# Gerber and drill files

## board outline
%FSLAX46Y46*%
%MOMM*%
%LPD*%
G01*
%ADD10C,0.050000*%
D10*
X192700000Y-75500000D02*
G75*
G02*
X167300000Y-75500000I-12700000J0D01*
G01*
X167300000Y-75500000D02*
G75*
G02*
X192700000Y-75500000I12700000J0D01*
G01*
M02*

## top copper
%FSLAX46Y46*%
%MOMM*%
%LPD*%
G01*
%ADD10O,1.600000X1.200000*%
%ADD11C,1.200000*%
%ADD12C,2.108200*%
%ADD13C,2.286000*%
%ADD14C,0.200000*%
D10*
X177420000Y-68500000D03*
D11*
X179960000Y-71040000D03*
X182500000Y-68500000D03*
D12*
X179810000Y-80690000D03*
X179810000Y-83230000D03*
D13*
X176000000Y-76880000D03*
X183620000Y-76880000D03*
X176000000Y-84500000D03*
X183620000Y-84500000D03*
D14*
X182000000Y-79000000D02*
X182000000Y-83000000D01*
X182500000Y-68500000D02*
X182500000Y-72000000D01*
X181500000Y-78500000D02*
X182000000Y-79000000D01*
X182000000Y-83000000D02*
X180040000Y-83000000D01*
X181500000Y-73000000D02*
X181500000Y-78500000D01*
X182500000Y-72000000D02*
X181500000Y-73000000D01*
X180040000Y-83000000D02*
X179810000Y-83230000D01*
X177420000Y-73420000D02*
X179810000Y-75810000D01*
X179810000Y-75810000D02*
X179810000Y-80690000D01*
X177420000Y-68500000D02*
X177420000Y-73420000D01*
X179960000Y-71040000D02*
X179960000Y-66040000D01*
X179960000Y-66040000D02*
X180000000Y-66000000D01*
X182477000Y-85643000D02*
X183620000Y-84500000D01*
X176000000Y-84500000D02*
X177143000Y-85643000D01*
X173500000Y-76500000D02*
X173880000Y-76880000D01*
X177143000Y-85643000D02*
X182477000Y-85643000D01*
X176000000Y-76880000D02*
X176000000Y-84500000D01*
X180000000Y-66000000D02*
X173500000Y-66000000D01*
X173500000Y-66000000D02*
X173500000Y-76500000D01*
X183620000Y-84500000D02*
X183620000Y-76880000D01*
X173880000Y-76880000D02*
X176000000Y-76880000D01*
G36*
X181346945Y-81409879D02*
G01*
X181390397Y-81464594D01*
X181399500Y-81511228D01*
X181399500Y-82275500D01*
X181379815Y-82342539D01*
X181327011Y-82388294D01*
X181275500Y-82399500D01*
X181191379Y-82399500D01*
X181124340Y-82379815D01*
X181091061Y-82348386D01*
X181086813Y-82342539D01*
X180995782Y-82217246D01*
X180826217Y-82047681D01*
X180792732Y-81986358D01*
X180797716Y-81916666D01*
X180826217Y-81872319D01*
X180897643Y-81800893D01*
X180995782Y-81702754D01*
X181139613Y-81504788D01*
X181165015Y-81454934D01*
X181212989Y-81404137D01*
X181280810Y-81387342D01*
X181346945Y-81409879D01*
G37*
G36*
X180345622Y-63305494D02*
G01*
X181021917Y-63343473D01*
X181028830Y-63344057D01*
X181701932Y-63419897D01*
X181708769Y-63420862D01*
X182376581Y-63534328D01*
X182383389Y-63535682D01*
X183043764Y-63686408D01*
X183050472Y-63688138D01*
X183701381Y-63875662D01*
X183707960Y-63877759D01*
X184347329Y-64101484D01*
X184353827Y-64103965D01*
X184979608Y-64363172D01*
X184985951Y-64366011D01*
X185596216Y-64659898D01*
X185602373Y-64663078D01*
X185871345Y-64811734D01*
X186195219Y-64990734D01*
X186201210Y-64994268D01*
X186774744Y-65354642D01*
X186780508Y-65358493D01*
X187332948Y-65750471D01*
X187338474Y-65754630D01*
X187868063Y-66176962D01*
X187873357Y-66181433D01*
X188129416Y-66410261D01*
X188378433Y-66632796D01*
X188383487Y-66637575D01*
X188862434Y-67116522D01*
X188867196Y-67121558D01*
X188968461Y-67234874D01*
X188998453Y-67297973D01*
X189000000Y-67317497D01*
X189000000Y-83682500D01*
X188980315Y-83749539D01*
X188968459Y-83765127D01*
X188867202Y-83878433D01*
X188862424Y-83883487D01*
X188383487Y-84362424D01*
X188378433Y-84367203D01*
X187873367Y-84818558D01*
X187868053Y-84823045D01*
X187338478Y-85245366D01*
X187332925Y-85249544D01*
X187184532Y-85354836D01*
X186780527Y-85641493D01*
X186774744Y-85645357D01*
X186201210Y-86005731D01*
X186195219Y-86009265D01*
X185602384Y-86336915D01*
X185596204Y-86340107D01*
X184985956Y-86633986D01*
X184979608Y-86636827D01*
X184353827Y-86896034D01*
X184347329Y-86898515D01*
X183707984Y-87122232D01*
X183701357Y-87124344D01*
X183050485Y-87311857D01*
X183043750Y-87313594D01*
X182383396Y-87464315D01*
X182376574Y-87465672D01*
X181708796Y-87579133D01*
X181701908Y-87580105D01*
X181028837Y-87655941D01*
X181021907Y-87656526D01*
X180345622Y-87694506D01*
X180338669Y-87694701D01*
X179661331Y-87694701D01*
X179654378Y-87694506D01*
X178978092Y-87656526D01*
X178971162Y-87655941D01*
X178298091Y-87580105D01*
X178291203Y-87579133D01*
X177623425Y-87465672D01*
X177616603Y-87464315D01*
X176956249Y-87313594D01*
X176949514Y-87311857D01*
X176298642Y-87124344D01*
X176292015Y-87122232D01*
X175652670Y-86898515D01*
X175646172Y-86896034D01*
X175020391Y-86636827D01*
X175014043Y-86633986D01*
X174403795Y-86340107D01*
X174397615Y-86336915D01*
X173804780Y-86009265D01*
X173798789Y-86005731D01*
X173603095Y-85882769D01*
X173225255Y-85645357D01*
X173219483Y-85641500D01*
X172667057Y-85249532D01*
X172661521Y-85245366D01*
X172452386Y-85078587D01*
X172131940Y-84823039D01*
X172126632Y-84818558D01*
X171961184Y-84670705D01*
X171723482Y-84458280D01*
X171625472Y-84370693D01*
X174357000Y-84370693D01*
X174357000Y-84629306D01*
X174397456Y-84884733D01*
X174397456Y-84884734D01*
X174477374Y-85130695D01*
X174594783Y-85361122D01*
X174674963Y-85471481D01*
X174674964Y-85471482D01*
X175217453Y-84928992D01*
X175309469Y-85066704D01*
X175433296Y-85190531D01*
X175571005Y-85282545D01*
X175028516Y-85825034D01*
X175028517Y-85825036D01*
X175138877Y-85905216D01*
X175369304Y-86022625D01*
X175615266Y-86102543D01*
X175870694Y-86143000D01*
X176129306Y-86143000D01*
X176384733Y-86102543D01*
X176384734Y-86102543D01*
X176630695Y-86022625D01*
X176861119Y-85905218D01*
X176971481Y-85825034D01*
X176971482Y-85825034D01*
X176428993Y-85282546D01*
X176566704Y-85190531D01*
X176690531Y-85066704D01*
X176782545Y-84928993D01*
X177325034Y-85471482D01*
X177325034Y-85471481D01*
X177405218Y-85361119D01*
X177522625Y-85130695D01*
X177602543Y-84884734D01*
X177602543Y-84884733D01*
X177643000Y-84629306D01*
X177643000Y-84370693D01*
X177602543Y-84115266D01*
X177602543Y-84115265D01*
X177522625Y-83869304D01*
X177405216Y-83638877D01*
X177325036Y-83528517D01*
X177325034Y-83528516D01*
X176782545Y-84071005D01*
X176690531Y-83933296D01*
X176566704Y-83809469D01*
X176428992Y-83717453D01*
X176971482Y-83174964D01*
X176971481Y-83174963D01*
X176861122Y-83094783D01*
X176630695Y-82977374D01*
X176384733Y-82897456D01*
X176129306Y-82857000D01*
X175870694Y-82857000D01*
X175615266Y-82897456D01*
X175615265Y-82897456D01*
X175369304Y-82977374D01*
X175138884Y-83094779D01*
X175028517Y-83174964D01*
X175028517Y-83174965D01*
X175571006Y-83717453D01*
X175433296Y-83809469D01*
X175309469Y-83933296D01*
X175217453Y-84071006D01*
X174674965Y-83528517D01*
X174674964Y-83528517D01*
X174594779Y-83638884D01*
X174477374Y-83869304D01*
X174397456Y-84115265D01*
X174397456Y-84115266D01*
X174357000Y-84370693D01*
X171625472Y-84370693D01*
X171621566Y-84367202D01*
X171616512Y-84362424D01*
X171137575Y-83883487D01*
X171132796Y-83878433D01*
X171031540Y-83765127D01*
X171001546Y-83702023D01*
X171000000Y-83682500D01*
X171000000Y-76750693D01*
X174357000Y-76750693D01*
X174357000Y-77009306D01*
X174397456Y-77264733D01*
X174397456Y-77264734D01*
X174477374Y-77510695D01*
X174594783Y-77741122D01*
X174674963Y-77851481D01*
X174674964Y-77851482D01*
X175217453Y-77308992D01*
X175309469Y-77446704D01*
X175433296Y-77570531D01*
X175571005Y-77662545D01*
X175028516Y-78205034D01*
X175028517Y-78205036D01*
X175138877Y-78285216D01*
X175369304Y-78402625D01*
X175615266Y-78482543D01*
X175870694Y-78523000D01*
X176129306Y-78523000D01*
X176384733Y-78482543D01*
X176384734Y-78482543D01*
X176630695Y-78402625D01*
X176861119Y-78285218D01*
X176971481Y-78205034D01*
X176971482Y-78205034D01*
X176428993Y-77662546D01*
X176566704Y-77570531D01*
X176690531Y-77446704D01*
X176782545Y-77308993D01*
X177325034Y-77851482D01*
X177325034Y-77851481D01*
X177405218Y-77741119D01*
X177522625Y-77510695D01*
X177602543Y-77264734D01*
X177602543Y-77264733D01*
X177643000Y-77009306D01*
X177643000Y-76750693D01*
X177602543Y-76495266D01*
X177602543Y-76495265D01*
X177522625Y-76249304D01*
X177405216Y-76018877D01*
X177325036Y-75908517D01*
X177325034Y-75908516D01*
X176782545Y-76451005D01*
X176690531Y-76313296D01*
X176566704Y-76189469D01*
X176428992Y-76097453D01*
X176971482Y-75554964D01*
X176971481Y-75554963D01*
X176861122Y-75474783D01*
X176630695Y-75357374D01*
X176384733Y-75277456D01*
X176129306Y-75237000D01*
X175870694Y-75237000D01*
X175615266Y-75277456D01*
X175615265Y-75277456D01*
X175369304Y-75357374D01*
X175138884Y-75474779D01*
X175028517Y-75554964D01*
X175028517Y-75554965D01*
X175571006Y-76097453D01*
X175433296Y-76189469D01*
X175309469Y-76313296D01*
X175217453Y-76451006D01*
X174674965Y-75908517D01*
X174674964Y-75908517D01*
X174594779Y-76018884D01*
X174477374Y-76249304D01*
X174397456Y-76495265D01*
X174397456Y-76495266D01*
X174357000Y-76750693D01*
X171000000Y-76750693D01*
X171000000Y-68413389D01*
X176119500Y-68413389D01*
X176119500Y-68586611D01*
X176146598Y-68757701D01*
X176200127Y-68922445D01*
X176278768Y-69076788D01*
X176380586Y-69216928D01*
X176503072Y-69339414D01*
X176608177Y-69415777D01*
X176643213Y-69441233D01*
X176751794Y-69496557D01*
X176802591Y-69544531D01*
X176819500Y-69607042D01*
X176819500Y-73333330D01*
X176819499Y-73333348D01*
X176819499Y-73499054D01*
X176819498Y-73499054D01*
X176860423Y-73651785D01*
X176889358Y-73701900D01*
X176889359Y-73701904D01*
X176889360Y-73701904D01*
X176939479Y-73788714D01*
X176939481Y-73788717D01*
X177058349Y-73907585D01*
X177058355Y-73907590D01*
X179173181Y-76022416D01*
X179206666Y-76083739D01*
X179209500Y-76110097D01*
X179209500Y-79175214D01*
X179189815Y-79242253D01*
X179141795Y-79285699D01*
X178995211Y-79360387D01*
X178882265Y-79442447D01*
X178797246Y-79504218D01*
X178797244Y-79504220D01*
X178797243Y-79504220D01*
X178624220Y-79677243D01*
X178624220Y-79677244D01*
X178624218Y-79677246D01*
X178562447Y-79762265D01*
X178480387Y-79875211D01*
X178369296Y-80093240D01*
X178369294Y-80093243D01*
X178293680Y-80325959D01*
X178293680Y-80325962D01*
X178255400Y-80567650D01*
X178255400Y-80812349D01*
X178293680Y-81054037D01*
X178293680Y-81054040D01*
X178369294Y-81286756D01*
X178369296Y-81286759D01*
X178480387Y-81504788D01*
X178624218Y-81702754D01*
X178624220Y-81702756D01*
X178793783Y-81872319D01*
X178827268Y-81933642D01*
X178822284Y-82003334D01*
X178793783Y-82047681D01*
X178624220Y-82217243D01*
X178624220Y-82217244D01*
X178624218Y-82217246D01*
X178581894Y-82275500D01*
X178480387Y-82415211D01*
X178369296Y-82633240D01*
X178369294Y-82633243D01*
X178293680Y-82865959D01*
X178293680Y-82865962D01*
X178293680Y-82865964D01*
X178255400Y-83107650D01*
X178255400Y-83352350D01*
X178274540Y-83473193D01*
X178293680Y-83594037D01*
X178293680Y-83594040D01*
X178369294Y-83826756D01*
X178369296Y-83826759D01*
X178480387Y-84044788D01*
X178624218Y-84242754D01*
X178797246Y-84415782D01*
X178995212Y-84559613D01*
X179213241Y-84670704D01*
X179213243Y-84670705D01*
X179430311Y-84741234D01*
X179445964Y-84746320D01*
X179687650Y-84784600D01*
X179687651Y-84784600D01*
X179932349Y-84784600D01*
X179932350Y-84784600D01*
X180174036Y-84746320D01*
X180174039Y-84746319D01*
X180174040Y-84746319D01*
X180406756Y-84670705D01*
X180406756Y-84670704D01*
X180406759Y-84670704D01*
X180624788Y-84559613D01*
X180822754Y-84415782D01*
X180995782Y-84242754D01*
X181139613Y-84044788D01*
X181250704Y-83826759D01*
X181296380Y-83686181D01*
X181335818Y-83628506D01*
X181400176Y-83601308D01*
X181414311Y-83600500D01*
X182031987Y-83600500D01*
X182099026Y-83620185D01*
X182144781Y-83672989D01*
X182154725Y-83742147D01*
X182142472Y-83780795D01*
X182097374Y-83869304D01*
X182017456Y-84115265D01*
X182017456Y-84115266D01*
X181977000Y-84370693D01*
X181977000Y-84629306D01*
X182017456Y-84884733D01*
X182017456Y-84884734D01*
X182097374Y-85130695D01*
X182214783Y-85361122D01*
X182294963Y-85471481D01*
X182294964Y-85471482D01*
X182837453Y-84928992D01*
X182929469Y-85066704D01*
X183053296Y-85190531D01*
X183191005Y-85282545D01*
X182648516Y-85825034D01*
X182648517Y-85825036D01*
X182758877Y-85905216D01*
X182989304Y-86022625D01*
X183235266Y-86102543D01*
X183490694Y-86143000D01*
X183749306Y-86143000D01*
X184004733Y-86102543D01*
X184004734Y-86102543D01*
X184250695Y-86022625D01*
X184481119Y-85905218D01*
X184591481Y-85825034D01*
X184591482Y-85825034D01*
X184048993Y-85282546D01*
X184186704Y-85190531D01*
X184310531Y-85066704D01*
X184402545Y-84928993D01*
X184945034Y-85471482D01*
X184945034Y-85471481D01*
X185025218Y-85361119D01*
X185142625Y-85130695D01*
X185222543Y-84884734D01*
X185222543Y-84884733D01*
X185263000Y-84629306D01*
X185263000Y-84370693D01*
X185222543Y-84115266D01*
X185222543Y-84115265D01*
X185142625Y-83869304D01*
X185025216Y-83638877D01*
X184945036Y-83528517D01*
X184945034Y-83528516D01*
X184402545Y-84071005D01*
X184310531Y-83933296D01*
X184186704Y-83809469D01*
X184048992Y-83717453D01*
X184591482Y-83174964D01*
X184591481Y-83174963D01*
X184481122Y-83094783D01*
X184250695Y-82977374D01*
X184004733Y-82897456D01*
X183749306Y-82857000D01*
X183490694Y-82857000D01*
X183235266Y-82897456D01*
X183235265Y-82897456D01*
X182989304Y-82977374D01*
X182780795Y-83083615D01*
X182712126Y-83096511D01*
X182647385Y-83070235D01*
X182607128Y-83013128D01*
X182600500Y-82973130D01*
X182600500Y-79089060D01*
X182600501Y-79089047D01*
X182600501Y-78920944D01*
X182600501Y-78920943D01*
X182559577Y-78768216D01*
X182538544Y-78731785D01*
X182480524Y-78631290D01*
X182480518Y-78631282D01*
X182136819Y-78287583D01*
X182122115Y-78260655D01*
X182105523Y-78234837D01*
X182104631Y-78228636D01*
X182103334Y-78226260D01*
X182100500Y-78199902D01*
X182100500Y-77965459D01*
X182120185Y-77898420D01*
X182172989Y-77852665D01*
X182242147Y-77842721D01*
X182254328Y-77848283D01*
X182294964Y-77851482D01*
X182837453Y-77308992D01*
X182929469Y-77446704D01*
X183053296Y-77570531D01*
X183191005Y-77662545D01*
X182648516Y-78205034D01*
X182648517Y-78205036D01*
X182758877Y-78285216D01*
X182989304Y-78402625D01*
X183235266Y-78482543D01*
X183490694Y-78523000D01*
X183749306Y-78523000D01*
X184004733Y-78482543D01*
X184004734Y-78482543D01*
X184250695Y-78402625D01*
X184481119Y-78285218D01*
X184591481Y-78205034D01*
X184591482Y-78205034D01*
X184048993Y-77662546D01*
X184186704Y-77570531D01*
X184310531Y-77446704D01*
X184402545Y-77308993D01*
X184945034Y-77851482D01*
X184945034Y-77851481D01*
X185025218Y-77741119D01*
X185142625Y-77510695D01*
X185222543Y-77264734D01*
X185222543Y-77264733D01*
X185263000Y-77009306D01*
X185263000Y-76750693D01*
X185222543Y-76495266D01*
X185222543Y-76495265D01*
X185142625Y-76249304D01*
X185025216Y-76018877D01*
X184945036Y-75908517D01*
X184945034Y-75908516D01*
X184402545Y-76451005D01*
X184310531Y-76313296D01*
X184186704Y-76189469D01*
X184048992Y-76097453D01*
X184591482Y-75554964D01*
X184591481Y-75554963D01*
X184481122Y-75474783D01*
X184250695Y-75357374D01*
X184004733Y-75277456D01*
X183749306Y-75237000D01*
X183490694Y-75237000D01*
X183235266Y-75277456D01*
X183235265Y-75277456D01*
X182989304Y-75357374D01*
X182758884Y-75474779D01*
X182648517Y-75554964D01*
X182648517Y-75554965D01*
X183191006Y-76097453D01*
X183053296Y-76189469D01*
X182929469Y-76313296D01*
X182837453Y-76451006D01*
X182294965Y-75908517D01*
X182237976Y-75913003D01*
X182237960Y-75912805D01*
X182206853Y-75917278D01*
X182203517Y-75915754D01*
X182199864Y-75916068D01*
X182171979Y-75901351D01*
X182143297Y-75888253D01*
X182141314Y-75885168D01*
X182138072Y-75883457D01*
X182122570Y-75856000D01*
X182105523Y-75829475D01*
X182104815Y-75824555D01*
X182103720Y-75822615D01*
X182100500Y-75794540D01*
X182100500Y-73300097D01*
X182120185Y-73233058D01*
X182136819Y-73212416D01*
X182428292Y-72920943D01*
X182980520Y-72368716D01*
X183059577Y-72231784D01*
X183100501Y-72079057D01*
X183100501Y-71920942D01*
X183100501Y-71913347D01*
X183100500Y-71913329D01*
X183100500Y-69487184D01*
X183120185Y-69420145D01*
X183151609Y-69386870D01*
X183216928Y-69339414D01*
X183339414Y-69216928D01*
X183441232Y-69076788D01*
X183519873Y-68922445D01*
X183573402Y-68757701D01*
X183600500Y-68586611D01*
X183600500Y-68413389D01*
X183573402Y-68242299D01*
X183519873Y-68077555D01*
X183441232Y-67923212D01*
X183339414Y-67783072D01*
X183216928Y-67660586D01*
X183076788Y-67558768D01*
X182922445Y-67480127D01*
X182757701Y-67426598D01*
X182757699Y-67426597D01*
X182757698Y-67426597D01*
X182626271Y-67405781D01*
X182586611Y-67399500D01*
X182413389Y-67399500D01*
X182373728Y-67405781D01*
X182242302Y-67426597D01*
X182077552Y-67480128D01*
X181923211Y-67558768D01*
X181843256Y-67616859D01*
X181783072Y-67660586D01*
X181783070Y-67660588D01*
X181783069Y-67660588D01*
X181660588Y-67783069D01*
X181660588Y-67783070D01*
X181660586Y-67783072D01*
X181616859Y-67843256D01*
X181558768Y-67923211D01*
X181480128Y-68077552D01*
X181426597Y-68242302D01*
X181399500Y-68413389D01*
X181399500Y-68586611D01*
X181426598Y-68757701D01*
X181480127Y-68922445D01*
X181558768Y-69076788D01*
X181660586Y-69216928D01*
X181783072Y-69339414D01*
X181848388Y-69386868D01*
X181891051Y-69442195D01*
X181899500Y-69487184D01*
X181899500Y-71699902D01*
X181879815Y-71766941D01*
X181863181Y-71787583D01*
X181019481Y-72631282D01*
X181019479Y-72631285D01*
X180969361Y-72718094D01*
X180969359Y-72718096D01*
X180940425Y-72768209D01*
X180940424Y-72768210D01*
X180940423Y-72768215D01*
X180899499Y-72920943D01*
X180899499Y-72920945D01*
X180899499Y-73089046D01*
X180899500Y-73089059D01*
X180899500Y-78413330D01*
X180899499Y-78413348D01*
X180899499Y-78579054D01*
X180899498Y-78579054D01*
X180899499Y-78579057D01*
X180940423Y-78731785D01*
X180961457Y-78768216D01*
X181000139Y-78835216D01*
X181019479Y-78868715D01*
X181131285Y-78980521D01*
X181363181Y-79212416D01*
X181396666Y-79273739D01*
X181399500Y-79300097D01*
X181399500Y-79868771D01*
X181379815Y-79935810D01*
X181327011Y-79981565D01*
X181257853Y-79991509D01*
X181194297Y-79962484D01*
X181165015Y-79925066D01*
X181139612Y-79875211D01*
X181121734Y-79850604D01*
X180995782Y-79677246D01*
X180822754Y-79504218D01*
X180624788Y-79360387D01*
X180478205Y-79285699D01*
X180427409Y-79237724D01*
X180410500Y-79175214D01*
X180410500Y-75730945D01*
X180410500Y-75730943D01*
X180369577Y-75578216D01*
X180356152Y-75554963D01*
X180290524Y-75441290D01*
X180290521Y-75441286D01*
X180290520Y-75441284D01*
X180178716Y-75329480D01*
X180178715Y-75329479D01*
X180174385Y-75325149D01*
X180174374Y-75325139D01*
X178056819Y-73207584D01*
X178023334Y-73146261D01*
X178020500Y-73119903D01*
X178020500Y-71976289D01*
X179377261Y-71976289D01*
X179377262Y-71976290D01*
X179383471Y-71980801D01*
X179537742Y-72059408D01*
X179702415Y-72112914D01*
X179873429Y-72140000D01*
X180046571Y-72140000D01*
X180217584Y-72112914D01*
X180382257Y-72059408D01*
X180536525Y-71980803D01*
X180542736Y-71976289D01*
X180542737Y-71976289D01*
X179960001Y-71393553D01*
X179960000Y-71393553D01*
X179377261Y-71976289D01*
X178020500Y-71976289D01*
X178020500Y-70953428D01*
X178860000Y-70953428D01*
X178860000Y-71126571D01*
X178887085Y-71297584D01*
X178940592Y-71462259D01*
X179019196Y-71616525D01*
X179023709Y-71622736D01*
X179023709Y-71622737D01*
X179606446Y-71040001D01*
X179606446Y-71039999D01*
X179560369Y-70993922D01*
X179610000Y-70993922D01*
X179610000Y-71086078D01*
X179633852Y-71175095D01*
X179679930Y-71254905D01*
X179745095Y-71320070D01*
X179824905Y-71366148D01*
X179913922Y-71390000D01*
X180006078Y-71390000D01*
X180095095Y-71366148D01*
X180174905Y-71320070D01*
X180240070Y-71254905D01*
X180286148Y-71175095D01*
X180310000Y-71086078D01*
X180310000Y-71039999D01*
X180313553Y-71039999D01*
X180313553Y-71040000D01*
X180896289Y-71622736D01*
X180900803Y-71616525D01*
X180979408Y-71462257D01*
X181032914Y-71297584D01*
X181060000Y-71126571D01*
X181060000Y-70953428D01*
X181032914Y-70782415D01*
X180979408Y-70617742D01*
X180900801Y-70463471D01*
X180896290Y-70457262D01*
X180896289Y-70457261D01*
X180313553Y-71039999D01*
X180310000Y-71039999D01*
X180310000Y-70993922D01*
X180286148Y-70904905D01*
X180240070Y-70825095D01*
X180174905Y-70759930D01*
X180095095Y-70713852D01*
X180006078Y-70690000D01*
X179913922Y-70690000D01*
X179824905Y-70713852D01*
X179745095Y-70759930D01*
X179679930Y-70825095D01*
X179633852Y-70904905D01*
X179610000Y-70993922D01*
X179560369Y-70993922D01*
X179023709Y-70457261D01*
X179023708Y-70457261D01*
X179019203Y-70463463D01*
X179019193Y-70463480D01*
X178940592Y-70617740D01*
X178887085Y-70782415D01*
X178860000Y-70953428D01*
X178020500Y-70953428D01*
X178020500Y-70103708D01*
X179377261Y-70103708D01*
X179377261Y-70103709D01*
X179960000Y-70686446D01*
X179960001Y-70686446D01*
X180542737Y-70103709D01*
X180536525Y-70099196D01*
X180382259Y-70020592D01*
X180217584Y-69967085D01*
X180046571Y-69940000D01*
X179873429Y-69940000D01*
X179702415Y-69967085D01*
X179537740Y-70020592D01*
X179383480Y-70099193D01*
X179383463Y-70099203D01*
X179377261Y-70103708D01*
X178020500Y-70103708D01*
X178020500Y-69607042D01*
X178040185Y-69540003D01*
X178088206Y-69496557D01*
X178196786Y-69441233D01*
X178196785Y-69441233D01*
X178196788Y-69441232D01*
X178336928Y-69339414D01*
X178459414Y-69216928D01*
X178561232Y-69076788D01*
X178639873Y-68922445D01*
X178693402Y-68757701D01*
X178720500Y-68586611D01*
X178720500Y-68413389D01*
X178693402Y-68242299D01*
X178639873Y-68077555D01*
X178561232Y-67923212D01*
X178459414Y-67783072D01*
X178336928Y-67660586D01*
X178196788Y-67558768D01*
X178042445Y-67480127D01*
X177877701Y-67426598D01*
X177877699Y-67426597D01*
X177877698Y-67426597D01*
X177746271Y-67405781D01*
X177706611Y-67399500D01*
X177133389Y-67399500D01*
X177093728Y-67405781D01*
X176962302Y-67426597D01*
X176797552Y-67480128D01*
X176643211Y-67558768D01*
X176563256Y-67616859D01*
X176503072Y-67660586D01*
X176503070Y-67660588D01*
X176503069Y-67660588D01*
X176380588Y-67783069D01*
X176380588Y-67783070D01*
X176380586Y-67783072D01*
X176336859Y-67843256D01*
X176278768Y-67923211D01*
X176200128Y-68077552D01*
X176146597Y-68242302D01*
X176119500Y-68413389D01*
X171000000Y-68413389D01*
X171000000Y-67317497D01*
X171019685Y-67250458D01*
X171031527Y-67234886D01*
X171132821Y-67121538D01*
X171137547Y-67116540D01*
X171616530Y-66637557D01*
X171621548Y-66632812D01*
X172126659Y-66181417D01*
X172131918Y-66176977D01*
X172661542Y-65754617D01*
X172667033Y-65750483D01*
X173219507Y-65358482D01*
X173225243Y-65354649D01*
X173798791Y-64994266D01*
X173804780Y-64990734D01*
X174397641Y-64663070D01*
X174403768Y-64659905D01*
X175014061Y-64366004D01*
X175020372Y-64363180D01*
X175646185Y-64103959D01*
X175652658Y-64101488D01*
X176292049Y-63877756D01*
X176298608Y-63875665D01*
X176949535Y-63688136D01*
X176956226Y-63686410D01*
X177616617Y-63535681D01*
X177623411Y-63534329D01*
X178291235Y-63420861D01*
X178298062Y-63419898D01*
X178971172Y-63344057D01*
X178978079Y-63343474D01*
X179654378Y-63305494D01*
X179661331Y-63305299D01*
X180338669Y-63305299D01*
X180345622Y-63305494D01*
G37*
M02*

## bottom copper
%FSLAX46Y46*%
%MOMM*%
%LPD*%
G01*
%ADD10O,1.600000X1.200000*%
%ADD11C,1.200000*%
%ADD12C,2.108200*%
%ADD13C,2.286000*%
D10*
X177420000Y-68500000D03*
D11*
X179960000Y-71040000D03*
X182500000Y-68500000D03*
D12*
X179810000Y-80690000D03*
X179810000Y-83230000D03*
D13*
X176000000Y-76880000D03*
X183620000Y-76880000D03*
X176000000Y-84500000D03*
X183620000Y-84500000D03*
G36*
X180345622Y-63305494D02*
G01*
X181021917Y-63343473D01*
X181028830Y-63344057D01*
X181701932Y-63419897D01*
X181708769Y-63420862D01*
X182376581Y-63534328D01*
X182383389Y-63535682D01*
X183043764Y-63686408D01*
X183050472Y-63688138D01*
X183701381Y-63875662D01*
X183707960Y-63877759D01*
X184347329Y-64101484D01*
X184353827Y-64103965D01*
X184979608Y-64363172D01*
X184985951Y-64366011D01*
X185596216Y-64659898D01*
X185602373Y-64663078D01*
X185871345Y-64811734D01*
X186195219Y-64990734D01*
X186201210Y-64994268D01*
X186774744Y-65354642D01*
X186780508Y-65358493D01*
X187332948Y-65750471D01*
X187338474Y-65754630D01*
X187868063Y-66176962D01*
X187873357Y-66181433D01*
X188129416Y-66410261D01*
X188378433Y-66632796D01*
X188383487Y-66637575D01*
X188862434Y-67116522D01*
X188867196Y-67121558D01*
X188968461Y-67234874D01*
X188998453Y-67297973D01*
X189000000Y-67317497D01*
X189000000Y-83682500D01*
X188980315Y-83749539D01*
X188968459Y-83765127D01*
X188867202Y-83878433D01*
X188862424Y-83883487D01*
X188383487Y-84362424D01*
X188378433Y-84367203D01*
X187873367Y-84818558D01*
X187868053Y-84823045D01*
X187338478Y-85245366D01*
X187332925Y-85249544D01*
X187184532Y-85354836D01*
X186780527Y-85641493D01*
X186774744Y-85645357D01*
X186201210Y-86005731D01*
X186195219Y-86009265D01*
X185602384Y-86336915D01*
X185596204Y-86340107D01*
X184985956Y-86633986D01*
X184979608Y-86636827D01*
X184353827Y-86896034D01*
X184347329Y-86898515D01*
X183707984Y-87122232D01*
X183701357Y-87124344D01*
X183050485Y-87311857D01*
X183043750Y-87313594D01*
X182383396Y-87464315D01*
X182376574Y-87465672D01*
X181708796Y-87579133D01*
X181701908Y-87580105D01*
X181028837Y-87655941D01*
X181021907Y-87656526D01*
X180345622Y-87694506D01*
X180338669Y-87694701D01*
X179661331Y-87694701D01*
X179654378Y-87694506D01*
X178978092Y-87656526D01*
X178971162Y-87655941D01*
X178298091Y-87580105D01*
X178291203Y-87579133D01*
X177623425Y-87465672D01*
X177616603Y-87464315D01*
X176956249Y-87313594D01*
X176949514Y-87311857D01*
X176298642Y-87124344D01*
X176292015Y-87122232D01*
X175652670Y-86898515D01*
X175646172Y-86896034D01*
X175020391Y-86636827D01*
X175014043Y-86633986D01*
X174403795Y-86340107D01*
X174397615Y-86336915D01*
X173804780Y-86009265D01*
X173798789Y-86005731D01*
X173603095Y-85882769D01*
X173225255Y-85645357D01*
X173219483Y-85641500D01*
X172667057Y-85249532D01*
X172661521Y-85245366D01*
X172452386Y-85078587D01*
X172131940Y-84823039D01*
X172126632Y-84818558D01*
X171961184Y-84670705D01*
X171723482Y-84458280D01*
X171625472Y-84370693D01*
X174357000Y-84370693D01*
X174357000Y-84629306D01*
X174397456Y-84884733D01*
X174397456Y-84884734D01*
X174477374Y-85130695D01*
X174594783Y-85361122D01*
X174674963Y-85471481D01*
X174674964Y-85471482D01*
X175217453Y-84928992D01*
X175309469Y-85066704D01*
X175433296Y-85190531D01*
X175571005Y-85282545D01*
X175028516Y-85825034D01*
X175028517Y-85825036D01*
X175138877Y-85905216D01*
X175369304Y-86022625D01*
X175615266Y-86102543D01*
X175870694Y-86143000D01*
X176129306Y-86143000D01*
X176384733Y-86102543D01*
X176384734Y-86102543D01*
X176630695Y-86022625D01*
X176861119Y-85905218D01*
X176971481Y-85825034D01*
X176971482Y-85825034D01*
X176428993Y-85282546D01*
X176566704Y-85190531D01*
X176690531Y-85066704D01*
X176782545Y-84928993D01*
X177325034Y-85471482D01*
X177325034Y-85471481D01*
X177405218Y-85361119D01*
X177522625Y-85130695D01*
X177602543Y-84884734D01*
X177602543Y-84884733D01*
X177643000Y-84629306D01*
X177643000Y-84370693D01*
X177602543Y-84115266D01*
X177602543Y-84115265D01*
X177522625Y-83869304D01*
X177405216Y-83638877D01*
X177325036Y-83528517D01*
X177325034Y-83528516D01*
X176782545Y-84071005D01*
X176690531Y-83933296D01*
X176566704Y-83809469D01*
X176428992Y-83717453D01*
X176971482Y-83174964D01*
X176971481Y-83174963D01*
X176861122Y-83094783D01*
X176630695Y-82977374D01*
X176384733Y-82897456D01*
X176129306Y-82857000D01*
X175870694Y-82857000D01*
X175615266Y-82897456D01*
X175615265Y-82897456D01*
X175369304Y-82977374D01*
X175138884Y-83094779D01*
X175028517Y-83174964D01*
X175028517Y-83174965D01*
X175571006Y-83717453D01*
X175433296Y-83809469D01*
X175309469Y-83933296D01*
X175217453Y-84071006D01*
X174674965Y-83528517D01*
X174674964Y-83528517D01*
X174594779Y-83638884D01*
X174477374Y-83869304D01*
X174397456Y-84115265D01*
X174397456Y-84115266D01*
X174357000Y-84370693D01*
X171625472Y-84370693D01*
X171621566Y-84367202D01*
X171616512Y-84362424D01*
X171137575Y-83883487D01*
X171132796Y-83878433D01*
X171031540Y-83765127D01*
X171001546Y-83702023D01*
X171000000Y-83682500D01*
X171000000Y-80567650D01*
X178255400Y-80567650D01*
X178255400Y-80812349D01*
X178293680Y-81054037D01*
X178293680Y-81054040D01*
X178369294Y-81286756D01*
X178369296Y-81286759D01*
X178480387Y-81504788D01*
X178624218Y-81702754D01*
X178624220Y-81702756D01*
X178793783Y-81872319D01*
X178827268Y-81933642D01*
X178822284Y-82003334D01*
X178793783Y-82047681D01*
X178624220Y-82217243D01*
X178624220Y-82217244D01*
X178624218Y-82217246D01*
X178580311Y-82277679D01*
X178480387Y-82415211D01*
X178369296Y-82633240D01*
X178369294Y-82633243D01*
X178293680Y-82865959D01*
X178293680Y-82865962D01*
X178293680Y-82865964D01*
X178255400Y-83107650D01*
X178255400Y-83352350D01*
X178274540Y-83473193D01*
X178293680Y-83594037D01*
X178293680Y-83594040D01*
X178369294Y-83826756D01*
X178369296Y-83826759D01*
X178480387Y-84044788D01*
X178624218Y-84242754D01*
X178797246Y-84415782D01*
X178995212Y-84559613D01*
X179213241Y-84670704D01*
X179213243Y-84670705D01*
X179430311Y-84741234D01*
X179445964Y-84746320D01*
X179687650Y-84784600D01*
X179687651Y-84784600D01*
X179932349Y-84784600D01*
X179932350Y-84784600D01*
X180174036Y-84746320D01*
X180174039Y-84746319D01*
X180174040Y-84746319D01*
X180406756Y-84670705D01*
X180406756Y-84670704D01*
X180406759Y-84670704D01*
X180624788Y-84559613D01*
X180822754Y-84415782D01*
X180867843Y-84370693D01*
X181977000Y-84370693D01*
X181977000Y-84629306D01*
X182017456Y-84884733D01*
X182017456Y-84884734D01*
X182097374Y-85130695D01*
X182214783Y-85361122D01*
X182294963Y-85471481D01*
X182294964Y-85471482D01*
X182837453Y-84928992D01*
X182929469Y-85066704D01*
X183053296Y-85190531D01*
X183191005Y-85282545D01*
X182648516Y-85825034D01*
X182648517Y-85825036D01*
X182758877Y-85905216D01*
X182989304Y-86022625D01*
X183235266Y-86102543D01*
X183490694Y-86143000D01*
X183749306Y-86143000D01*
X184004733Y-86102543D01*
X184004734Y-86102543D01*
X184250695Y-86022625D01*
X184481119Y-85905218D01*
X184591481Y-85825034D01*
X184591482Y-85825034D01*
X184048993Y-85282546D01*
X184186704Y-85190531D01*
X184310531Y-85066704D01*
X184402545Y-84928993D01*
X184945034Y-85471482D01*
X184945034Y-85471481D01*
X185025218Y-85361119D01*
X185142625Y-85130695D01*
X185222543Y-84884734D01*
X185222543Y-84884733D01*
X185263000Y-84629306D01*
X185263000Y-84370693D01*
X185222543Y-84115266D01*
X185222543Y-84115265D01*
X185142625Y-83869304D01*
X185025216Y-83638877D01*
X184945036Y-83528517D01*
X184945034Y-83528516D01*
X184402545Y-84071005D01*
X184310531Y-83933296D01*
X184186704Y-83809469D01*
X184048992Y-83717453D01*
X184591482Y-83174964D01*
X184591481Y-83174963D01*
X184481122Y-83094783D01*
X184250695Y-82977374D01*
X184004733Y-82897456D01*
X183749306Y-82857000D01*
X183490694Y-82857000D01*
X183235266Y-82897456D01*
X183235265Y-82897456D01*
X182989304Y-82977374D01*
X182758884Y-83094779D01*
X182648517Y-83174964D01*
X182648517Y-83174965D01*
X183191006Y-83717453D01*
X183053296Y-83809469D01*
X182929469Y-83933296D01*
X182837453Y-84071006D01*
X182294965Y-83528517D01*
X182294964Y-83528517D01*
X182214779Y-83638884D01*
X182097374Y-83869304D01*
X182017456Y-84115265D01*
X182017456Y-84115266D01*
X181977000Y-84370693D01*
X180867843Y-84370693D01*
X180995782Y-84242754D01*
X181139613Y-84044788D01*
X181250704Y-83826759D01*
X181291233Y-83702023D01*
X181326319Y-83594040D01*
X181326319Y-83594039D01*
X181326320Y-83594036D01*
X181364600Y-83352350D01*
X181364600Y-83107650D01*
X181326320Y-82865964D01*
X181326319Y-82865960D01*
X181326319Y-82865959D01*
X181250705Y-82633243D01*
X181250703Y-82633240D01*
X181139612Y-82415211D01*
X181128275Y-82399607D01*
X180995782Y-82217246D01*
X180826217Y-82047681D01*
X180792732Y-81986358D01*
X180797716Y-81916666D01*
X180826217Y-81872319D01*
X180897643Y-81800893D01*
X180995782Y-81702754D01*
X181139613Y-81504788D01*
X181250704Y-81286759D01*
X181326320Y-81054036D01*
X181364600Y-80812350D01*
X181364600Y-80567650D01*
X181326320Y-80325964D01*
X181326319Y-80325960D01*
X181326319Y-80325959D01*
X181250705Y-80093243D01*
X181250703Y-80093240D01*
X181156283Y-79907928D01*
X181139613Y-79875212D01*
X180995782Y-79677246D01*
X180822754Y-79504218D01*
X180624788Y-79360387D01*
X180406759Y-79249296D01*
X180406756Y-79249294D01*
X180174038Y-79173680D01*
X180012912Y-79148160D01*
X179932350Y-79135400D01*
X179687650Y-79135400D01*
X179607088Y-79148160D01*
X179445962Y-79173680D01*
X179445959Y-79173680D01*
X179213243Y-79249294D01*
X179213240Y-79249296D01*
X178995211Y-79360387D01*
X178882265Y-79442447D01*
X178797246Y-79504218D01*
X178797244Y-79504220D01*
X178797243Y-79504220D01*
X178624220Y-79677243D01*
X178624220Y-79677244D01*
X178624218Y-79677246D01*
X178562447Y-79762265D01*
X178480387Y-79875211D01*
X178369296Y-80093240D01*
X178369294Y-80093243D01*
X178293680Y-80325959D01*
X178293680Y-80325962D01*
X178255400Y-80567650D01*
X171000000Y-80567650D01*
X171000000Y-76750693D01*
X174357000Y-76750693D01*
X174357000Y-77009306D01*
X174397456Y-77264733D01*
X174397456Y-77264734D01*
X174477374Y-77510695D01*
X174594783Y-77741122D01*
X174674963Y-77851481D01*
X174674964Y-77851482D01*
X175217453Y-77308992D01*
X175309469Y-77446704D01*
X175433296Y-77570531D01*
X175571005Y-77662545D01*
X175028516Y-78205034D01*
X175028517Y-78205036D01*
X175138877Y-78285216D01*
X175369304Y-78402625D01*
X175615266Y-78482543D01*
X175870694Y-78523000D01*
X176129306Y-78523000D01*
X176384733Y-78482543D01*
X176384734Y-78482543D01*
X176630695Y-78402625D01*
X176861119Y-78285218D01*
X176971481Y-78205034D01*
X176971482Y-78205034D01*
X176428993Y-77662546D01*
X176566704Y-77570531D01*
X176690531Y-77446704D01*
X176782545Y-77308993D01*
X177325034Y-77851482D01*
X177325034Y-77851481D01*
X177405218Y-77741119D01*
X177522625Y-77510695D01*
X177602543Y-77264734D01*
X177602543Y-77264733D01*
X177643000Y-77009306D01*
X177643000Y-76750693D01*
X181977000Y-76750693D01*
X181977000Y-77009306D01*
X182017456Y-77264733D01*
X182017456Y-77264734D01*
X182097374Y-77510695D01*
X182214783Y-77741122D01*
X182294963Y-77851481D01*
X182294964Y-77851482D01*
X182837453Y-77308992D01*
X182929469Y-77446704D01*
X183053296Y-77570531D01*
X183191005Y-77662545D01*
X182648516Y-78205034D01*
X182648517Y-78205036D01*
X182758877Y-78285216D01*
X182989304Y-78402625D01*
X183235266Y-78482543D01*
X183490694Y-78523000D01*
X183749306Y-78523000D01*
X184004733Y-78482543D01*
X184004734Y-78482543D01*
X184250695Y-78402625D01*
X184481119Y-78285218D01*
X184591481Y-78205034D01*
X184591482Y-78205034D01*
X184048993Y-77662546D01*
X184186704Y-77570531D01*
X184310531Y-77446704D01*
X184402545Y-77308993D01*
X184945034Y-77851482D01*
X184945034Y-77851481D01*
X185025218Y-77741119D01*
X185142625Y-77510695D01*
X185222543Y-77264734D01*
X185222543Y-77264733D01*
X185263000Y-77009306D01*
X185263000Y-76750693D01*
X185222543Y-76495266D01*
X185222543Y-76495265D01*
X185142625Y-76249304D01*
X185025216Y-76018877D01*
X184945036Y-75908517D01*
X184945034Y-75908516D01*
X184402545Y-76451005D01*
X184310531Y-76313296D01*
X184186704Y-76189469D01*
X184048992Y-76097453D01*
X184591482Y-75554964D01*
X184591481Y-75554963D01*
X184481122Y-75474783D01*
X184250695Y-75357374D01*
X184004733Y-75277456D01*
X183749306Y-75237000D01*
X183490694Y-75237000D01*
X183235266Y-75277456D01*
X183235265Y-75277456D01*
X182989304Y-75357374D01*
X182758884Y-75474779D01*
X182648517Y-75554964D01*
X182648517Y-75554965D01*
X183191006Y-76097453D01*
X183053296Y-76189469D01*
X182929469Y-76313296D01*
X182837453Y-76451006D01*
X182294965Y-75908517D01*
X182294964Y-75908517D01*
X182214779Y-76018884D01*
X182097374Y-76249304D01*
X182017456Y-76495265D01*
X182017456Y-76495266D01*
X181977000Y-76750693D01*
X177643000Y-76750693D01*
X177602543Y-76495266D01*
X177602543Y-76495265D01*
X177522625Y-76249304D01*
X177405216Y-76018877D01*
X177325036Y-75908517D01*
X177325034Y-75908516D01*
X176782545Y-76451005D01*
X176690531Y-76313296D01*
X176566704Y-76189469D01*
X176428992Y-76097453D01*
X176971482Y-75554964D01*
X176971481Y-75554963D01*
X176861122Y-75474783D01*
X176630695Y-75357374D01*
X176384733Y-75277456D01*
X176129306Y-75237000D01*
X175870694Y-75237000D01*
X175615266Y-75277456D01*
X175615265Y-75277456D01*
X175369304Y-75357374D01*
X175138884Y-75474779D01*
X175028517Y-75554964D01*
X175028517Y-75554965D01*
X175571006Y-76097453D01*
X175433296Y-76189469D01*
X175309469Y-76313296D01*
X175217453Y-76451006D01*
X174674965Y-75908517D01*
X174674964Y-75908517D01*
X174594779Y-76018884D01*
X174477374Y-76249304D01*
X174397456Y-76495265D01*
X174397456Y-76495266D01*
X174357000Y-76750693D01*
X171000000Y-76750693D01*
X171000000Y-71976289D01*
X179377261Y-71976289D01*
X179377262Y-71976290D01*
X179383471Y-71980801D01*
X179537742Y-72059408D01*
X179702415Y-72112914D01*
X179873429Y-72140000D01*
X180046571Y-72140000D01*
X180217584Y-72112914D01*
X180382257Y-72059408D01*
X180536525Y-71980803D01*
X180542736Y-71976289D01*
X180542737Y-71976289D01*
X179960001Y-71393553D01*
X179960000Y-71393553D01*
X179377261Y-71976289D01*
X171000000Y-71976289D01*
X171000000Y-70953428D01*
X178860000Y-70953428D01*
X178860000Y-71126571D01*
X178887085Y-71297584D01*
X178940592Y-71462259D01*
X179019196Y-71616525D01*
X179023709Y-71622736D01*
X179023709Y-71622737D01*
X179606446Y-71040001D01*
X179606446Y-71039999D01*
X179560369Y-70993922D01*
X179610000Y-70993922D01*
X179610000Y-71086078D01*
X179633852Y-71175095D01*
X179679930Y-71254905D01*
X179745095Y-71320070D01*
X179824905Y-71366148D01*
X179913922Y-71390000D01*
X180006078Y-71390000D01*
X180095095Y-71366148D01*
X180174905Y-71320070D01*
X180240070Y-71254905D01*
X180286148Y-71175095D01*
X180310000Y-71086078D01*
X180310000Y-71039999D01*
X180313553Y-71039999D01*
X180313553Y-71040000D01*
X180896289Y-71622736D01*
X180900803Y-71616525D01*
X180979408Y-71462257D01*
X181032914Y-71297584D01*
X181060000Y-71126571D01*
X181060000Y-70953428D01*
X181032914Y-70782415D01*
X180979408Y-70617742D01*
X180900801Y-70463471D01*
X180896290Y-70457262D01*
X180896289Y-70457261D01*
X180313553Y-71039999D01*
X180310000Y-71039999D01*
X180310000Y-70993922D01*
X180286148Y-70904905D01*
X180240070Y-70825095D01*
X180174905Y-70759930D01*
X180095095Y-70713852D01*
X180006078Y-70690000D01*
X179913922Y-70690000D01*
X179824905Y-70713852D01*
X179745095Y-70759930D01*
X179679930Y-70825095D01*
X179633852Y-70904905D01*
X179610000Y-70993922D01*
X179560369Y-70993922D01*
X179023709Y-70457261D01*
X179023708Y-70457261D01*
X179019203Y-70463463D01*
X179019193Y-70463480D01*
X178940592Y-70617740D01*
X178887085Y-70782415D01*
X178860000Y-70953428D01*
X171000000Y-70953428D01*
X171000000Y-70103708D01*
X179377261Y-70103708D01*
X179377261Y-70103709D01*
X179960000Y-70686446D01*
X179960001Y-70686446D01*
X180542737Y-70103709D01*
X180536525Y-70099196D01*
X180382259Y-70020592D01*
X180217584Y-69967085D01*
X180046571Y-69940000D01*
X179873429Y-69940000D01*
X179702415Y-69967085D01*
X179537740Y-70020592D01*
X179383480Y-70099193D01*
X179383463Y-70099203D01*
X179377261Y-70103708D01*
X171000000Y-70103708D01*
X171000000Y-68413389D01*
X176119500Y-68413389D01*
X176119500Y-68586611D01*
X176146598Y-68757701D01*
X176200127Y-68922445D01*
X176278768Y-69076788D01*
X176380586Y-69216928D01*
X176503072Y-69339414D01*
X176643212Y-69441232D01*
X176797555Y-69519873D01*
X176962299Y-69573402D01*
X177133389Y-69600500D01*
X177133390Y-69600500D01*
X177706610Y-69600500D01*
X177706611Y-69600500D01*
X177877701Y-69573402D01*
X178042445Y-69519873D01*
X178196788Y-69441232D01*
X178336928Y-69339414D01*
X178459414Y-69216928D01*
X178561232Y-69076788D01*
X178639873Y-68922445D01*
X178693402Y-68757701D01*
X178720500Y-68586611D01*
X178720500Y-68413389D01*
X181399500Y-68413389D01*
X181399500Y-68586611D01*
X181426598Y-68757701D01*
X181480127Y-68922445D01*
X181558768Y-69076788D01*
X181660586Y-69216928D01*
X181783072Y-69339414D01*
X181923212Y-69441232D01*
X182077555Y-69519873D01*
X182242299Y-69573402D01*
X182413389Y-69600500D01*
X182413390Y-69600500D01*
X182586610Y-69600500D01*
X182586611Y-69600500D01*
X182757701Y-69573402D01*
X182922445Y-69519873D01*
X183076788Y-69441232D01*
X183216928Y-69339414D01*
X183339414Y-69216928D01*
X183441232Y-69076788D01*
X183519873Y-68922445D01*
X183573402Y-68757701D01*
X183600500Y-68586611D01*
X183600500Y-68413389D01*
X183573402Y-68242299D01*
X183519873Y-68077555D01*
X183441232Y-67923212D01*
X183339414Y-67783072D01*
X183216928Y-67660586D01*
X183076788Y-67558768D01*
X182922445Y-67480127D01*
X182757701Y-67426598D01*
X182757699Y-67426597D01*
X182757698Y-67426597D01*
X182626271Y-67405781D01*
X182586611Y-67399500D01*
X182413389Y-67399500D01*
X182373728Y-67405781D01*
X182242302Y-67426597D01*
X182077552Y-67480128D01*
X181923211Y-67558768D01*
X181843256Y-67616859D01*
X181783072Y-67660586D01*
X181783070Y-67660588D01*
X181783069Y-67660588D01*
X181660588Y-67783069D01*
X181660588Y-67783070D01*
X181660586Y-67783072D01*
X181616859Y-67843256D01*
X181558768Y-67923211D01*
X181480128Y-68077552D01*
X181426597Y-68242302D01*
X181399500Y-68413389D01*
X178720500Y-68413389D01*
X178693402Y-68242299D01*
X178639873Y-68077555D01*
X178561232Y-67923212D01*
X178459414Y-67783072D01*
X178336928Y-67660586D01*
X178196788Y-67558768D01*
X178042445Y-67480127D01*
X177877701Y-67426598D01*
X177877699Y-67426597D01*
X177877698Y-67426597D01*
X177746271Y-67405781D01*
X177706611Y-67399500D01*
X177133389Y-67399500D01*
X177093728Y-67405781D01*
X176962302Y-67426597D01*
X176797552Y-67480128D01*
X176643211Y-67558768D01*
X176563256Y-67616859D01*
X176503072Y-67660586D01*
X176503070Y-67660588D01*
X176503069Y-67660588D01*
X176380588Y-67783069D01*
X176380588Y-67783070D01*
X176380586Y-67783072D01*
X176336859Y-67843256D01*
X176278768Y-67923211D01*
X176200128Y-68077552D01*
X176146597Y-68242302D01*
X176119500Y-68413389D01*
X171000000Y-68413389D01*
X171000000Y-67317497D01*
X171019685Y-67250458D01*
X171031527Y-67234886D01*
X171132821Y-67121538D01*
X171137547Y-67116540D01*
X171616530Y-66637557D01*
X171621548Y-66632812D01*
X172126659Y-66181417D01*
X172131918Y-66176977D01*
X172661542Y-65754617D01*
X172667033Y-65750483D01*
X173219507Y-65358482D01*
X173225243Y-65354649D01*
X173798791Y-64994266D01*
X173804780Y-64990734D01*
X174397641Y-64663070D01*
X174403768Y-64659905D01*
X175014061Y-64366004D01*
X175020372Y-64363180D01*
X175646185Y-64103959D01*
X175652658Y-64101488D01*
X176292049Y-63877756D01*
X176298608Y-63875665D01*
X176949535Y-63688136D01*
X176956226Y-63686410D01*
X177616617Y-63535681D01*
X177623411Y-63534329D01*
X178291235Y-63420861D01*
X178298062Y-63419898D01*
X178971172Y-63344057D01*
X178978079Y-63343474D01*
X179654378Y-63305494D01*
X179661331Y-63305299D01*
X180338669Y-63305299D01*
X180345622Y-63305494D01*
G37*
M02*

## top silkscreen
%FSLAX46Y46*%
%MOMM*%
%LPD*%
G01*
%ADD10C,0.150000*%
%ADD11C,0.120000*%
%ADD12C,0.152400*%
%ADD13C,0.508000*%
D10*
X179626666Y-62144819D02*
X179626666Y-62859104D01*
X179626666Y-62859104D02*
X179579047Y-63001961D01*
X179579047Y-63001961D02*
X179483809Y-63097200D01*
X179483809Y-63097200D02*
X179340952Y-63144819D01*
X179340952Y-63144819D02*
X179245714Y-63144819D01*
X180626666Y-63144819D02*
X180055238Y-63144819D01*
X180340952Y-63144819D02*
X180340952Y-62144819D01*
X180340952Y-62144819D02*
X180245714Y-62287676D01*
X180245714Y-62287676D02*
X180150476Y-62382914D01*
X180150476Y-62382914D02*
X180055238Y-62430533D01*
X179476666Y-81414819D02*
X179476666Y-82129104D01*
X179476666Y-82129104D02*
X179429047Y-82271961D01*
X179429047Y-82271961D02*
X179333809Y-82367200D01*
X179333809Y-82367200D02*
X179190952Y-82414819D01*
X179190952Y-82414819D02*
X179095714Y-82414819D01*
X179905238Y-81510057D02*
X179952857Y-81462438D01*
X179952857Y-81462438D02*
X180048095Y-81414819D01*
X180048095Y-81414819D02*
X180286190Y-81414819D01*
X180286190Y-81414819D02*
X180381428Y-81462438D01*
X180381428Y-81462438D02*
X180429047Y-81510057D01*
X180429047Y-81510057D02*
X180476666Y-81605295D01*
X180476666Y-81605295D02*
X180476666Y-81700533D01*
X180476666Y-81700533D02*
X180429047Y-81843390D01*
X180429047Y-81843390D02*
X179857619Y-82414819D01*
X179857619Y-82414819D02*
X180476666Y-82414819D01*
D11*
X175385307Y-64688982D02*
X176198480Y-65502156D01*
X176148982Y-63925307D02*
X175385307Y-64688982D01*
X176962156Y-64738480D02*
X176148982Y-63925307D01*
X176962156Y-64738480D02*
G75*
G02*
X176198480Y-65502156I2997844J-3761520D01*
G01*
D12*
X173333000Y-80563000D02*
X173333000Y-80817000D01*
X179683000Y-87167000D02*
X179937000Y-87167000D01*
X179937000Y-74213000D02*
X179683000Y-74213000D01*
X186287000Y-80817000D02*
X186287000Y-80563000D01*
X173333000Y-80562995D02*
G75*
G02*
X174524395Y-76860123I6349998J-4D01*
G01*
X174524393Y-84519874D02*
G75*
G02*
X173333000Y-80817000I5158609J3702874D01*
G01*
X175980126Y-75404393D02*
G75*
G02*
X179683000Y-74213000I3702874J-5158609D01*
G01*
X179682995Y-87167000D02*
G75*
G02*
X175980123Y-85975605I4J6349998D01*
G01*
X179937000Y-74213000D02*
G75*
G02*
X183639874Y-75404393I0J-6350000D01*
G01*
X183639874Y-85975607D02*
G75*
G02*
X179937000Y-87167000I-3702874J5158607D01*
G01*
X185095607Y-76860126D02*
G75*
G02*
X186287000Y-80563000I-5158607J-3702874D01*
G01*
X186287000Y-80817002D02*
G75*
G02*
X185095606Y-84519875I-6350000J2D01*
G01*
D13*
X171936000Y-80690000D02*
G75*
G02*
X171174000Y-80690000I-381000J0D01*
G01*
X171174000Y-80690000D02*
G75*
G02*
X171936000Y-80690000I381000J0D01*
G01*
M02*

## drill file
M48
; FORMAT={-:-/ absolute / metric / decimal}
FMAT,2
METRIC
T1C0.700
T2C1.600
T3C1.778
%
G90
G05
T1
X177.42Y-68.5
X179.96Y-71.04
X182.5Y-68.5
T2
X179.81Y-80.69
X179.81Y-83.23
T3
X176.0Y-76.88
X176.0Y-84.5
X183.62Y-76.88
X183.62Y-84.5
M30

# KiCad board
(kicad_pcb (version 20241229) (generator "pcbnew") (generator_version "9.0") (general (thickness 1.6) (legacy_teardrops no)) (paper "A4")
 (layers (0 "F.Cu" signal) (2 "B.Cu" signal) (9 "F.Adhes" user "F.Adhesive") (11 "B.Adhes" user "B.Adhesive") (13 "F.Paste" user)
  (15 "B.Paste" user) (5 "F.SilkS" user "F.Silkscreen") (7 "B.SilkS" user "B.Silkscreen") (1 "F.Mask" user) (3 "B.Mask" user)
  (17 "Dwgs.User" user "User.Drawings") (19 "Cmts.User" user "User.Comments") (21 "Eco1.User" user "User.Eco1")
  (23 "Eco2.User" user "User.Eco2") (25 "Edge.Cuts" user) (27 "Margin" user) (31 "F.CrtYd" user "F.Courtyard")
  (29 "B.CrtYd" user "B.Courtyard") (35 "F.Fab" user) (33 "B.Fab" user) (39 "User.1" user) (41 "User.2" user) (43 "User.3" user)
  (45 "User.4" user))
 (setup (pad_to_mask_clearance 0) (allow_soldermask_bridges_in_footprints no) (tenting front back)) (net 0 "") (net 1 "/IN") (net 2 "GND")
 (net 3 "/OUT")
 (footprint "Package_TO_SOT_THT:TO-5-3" (layer "F.Cu") (at 177.42 68.5)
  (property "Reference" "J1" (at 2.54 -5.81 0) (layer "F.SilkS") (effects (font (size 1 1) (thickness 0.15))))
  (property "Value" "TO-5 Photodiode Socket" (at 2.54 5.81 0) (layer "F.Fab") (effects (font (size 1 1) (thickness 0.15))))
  (fp_line (start -2.034693 -3.811018) (end -1.22152 -2.997844) (stroke (width 0.12) (type solid)) (layer "F.SilkS"))
  (fp_line (start -1.271018 -4.574693) (end -2.034693 -3.811018) (stroke (width 0.12) (type solid)) (layer "F.SilkS"))
  (fp_line (start -0.457844 -3.76152) (end -1.271018 -4.574693) (stroke (width 0.12) (type solid)) (layer "F.SilkS"))
  (fp_arc (start -0.457844 -3.76152) (mid 5.941184 3.401184) (end -1.22152 -2.997844) (stroke (width 0.12) (type solid)) (layer "F.SilkS"))
  (pad "1" thru_hole oval (at 0 0) (size 1.6 1.2) (drill 0.7) (layers "*.Cu" "*.Mask") (remove_unused_layers no) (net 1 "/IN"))
  (pad "2" thru_hole circle (at 2.54 2.54) (size 1.2 1.2) (drill 0.7) (layers "*.Cu" "*.Mask") (remove_unused_layers no) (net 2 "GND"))
  (pad "3" thru_hole circle (at 5.08 0) (size 1.2 1.2) (drill 0.7) (layers "*.Cu" "*.Mask") (remove_unused_layers no) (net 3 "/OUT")))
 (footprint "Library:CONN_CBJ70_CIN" (layer "F.Cu") (at 179.81 80.69)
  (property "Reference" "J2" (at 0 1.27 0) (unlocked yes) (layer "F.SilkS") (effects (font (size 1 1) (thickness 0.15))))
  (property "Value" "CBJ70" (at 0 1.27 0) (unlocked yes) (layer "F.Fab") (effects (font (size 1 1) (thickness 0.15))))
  (fp_line (start -6.477 -0.127) (end -6.477 0.127) (stroke (width 0.1524) (type solid)) (layer "F.SilkS"))
  (fp_line (start -0.127 6.477) (end 0.127 6.477) (stroke (width 0.1524) (type solid)) (layer "F.SilkS"))
  (fp_line (start 0.127 -6.477) (end -0.127 -6.477) (stroke (width 0.1524) (type solid)) (layer "F.SilkS"))
  (fp_line (start 6.477 0.127) (end 6.477 -0.127) (stroke (width 0.1524) (type solid)) (layer "F.SilkS"))
  (fp_arc (start -6.477 -0.127005) (mid -6.171817 -2.071914) (end -5.285605 -3.829877) (stroke (width 0.1524) (type solid))
   (layer "F.SilkS"))
  (fp_arc (start -5.285607 3.829874) (mid -6.171818 2.07191) (end -6.477 0.127) (stroke (width 0.1524) (type solid)) (layer "F.SilkS"))
  (fp_arc (start -3.829874 -5.285607) (mid -2.07191 -6.171818) (end -0.127 -6.477) (stroke (width 0.1524) (type solid)) (layer "F.SilkS"))
  (fp_arc (start -0.127005 6.477) (mid -2.071914 6.171817) (end -3.829877 5.285605) (stroke (width 0.1524) (type solid)) (layer "F.SilkS"))
  (fp_arc (start 0.127 -6.477) (mid 2.07191 -6.171818) (end 3.829874 -5.285607) (stroke (width 0.1524) (type solid)) (layer "F.SilkS"))
  (fp_arc (start 3.829874 5.285607) (mid 2.07191 6.171818) (end 0.127 6.477) (stroke (width 0.1524) (type solid)) (layer "F.SilkS"))
  (fp_arc (start 5.285607 -3.829874) (mid 6.171818 -2.07191) (end 6.477 -0.127) (stroke (width 0.1524) (type solid)) (layer "F.SilkS"))
  (fp_arc (start 6.477 0.127002) (mid 6.171818 2.071911) (end 5.285606 3.829875) (stroke (width 0.1524) (type solid)) (layer "F.SilkS"))
  (fp_circle (center -8.255 0) (end -7.874 0) (stroke (width 0.508) (type solid)) (fill no) (layer "F.SilkS"))
  (pad "1" thru_hole circle (at 0 0) (size 2.1082 2.1082) (drill 1.6002) (layers "*.Cu" "*.Mask") (remove_unused_layers no) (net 1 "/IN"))
  (pad "2" thru_hole circle (at 0 2.54) (size 2.1082 2.1082) (drill 1.6002) (layers "*.Cu" "*.Mask") (remove_unused_layers no)
   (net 3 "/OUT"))
  (pad "3" thru_hole circle (at -3.81 -3.81) (size 2.286 2.286) (drill 1.778) (layers "*.Cu" "*.Mask") (remove_unused_layers no)
   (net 2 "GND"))
  (pad "4" thru_hole circle (at 3.81 -3.81) (size 2.286 2.286) (drill 1.778) (layers "*.Cu" "*.Mask") (remove_unused_layers no)
   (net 2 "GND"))
  (pad "5" thru_hole circle (at -3.81 3.81) (size 2.286 2.286) (drill 1.778) (layers "*.Cu" "*.Mask") (remove_unused_layers no)
   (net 2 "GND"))
  (pad "6" thru_hole circle (at 3.81 3.81) (size 2.286 2.286) (drill 1.778) (layers "*.Cu" "*.Mask") (remove_unused_layers no) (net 2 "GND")))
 (gr_circle (center 180 75.5) (end 192.7 75.5) (stroke (width 0.05) (type solid)) (fill no) (layer "Edge.Cuts"))
 (segment (start 182 79) (end 182 83) (width 0.2) (layer "F.Cu") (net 3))
 (segment (start 182.5 68.5) (end 182.5 72) (width 0.2) (layer "F.Cu") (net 3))
 (segment (start 181.5 78.5) (end 182 79) (width 0.2) (layer "F.Cu") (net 3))
 (segment (start 182 83) (end 180.04 83) (width 0.2) (layer "F.Cu") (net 3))
 (segment (start 181.5 73) (end 181.5 78.5) (width 0.2) (layer "F.Cu") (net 3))
 (segment (start 182.5 72) (end 181.5 73) (width 0.2) (layer "F.Cu") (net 3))
 (segment (start 180.04 83) (end 179.81 83.23) (width 0.2) (layer "F.Cu") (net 3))
 (segment (start 177.42 73.42) (end 179.81 75.81) (width 0.2) (layer "F.Cu") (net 1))
 (segment (start 179.81 75.81) (end 179.81 80.69) (width 0.2) (layer "F.Cu") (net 1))
 (segment (start 177.42 68.5) (end 177.42 73.42) (width 0.2) (layer "F.Cu") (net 1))
 (segment (start 179.96 71.04) (end 179.96 66.04) (width 0.2) (layer "F.Cu") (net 2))
 (segment (start 179.96 66.04) (end 180 66) (width 0.2) (layer "F.Cu") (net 2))
 (segment (start 182.477 85.643) (end 183.62 84.5) (width 0.2) (layer "F.Cu") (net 2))
 (segment (start 176 84.5) (end 177.143 85.643) (width 0.2) (layer "F.Cu") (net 2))
 (segment (start 173.5 76.5) (end 173.88 76.88) (width 0.2) (layer "F.Cu") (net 2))
 (segment (start 177.143 85.643) (end 182.477 85.643) (width 0.2) (layer "F.Cu") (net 2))
 (segment (start 176 76.88) (end 176 84.5) (width 0.2) (layer "F.Cu") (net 2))
 (segment (start 180 66) (end 173.5 66) (width 0.2) (layer "F.Cu") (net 2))
 (segment (start 173.5 66) (end 173.5 76.5) (width 0.2) (layer "F.Cu") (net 2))
 (segment (start 183.62 84.5) (end 183.62 76.88) (width 0.2) (layer "F.Cu") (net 2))
 (segment (start 173.88 76.88) (end 176 76.88) (width 0.2) (layer "F.Cu") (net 2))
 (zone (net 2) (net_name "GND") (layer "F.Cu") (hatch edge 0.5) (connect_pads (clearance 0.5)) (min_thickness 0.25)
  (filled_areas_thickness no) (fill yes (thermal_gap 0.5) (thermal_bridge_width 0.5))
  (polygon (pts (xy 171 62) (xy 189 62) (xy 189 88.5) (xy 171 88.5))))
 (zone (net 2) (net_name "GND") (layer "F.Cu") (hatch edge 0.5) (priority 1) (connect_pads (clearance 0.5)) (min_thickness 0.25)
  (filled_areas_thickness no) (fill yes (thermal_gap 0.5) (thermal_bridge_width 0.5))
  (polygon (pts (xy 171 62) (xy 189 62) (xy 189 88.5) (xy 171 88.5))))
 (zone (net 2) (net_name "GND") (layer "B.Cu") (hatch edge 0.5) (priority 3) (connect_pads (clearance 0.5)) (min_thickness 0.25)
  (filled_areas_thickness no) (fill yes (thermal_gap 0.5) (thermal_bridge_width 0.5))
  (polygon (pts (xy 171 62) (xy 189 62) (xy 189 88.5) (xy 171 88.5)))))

